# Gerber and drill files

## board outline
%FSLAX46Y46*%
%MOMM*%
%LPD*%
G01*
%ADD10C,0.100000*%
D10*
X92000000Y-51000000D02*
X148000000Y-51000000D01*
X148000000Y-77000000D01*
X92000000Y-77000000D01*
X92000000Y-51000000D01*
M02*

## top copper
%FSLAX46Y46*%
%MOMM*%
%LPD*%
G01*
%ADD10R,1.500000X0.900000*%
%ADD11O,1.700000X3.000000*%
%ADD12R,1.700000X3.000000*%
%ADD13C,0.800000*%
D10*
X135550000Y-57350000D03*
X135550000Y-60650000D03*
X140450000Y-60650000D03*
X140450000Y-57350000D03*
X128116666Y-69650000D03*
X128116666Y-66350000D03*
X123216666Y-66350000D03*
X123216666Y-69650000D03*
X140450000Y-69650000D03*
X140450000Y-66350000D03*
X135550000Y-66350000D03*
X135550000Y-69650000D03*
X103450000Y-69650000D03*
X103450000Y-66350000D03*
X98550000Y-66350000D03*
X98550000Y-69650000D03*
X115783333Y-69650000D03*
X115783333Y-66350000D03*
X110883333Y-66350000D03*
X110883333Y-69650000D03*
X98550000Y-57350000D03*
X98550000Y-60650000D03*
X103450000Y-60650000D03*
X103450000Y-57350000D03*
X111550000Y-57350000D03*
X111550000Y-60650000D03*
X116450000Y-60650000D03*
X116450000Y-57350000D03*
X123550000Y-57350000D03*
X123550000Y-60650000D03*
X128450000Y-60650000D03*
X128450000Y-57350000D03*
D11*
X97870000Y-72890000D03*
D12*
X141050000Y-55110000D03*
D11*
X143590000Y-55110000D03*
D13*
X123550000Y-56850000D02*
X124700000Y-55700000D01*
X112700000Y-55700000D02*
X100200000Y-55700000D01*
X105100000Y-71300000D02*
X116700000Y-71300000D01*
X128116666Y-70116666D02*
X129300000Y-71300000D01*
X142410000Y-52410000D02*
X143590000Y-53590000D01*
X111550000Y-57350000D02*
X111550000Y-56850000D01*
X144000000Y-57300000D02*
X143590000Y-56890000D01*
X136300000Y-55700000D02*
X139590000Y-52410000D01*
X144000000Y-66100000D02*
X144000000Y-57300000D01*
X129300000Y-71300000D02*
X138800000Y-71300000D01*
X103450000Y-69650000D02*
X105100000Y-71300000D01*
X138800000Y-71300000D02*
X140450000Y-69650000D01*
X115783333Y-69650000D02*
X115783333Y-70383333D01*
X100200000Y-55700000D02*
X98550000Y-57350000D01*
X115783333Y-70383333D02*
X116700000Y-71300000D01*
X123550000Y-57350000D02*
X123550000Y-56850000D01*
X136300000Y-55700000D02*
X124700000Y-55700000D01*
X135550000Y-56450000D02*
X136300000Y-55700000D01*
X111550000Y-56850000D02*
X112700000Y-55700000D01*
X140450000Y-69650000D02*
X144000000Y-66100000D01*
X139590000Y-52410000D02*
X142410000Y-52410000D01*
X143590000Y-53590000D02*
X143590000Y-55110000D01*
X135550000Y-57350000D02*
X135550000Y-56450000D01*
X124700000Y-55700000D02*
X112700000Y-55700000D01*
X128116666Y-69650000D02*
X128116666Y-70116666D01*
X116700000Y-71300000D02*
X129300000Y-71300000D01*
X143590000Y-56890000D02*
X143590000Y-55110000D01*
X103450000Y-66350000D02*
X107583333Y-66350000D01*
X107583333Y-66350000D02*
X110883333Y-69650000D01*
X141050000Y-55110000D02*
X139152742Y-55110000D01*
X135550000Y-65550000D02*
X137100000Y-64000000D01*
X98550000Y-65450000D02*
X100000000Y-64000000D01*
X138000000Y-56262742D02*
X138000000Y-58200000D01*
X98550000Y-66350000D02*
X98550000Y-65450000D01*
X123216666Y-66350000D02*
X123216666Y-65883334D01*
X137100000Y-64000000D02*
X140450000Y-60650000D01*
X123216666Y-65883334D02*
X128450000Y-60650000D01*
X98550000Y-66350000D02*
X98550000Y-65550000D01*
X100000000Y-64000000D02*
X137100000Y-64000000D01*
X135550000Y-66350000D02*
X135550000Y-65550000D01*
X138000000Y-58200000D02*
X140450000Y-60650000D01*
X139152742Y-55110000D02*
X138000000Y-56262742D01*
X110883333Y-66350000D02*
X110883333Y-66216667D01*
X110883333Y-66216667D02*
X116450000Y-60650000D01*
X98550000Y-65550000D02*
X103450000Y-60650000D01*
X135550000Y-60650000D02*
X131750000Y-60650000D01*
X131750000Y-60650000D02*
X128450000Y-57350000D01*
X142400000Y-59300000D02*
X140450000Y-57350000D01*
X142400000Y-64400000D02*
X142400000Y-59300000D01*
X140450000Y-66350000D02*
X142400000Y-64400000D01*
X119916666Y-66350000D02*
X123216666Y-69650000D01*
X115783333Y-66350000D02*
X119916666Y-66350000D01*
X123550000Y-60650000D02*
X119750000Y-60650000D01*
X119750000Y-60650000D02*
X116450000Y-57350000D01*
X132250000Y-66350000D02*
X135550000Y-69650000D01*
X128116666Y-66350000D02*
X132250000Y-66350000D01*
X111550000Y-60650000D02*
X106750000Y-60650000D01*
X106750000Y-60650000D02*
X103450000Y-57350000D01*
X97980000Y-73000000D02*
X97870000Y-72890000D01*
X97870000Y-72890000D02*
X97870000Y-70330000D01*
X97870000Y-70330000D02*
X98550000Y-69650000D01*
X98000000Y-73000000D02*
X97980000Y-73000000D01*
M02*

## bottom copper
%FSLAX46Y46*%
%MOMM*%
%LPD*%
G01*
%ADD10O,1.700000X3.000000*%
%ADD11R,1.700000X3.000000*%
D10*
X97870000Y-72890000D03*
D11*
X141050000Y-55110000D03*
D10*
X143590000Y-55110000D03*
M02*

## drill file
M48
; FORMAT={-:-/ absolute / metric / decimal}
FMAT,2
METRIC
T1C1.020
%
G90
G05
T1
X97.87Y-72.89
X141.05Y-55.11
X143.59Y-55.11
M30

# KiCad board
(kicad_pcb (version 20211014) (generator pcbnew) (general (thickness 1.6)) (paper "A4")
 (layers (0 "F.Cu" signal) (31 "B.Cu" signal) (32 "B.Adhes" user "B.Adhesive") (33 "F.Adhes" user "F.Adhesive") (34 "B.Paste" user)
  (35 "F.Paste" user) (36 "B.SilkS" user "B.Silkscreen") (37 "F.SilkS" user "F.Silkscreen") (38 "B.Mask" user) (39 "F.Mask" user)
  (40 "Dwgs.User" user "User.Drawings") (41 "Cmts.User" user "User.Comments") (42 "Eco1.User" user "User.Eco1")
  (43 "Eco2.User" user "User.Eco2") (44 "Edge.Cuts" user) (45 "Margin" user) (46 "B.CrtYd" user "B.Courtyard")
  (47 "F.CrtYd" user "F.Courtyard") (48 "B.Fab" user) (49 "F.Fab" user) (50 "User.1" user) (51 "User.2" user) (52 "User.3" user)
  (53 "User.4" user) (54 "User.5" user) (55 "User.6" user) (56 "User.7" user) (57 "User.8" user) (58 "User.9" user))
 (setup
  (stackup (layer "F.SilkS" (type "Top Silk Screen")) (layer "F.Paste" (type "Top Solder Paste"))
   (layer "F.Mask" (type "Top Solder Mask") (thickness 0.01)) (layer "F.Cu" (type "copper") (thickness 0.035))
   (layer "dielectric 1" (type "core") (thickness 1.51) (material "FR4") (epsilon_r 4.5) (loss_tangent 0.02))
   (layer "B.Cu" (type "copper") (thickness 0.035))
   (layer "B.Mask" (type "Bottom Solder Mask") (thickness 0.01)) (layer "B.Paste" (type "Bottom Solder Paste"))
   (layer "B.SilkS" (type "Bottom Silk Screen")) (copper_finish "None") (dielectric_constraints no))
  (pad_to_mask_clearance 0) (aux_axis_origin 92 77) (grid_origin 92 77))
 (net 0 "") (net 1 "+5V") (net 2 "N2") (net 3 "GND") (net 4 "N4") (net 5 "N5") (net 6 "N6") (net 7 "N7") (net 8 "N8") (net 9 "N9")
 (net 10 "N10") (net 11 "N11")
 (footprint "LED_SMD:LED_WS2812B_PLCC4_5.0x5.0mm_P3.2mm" (layer "F.Cu") (at 138 59)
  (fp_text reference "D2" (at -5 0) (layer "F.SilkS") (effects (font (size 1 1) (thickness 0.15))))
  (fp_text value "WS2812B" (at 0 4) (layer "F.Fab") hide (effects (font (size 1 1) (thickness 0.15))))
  (pad "1" smd rect (at -2.45 -1.65) (size 1.5 0.9) (layers "F.Cu" "F.Paste" "F.Mask") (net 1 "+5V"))
  (pad "2" smd rect (at -2.45 1.65) (size 1.5 0.9) (layers "F.Cu" "F.Paste" "F.Mask") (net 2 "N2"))
  (pad "3" smd rect (at 2.45 1.65) (size 1.5 0.9) (layers "F.Cu" "F.Paste" "F.Mask") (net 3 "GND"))
  (pad "4" smd rect (at 2.45 -1.65) (size 1.5 0.9) (layers "F.Cu" "F.Paste" "F.Mask") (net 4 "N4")))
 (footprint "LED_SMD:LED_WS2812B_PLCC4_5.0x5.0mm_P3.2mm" (layer "F.Cu") (at 125.666666 68 180)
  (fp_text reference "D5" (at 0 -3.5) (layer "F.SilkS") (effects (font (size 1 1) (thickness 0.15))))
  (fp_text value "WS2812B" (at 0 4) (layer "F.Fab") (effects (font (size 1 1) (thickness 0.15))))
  (pad "1" smd rect (at -2.45 -1.65 180) (size 1.5 0.9) (layers "F.Cu" "F.Paste" "F.Mask") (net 1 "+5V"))
  (pad "2" smd rect (at -2.45 1.65 180) (size 1.5 0.9) (layers "F.Cu" "F.Paste" "F.Mask") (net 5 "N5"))
  (pad "3" smd rect (at 2.45 1.65 180) (size 1.5 0.9) (layers "F.Cu" "F.Paste" "F.Mask") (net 3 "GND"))
  (pad "4" smd rect (at 2.45 -1.65 180) (size 1.5 0.9) (layers "F.Cu" "F.Paste" "F.Mask") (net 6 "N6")))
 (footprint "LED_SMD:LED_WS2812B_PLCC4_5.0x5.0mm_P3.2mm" (layer "F.Cu") (at 138 68 180)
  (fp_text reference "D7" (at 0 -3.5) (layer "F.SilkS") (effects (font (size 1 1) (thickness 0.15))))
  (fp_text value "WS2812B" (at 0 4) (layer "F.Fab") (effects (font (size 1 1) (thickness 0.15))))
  (pad "1" smd rect (at -2.45 -1.65 180) (size 1.5 0.9) (layers "F.Cu" "F.Paste" "F.Mask") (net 1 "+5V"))
  (pad "2" smd rect (at -2.45 1.65 180) (size 1.5 0.9) (layers "F.Cu" "F.Paste" "F.Mask") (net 4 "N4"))
  (pad "3" smd rect (at 2.45 1.65 180) (size 1.5 0.9) (layers "F.Cu" "F.Paste" "F.Mask") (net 3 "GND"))
  (pad "4" smd rect (at 2.45 -1.65 180) (size 1.5 0.9) (layers "F.Cu" "F.Paste" "F.Mask") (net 5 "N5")))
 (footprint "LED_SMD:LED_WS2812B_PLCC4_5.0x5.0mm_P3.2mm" (layer "F.Cu") (at 101 68 180)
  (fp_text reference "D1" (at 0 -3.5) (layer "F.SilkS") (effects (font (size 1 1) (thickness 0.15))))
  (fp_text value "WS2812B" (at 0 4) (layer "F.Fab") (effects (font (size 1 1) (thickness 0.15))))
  (pad "1" smd rect (at -2.45 -1.65 180) (size 1.5 0.9) (layers "F.Cu" "F.Paste" "F.Mask") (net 1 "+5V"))
  (pad "2" smd rect (at -2.45 1.65 180) (size 1.5 0.9) (layers "F.Cu" "F.Paste" "F.Mask") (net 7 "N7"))
  (pad "3" smd rect (at 2.45 1.65 180) (size 1.5 0.9) (layers "F.Cu" "F.Paste" "F.Mask") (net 3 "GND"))
  (pad "4" smd rect (at 2.45 -1.65 180) (size 1.5 0.9) (layers "F.Cu" "F.Paste" "F.Mask") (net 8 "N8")))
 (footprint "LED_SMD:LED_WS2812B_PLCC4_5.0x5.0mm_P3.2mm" (layer "F.Cu") (at 113.333333 68 180)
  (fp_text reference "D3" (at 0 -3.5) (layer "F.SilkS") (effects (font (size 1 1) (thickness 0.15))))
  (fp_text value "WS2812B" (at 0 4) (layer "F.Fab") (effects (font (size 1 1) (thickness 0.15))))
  (pad "1" smd rect (at -2.45 -1.65 180) (size 1.5 0.9) (layers "F.Cu" "F.Paste" "F.Mask") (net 1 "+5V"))
  (pad "2" smd rect (at -2.45 1.65 180) (size 1.5 0.9) (layers "F.Cu" "F.Paste" "F.Mask") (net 6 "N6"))
  (pad "3" smd rect (at 2.45 1.65 180) (size 1.5 0.9) (layers "F.Cu" "F.Paste" "F.Mask") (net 3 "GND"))
  (pad "4" smd rect (at 2.45 -1.65 180) (size 1.5 0.9) (layers "F.Cu" "F.Paste" "F.Mask") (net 7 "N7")))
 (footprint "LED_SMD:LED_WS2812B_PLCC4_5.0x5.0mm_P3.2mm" (layer "F.Cu") (at 101 59)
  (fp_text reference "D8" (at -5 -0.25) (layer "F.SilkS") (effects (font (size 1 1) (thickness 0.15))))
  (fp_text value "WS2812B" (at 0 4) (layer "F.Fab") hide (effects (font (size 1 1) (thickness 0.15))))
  (pad "1" smd rect (at -2.45 -1.65) (size 1.5 0.9) (layers "F.Cu" "F.Paste" "F.Mask") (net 1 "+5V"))
  (pad "2" smd rect (at -2.45 1.65) (size 1.5 0.9) (layers "F.Cu" "F.Paste" "F.Mask") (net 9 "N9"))
  (pad "3" smd rect (at 2.45 1.65) (size 1.5 0.9) (layers "F.Cu" "F.Paste" "F.Mask") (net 3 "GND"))
  (pad "4" smd rect (at 2.45 -1.65) (size 1.5 0.9) (layers "F.Cu" "F.Paste" "F.Mask") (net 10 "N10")))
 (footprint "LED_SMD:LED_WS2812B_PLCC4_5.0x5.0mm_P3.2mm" (layer "F.Cu") (at 114 59)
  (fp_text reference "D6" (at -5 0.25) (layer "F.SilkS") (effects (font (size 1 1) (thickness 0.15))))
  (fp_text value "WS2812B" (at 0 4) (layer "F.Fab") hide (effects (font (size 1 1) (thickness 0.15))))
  (pad "1" smd rect (at -2.45 -1.65) (size 1.5 0.9) (layers "F.Cu" "F.Paste" "F.Mask") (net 1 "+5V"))
  (pad "2" smd rect (at -2.45 1.65) (size 1.5 0.9) (layers "F.Cu" "F.Paste" "F.Mask") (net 10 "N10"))
  (pad "3" smd rect (at 2.45 1.65) (size 1.5 0.9) (layers "F.Cu" "F.Paste" "F.Mask") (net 3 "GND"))
  (pad "4" smd rect (at 2.45 -1.65) (size 1.5 0.9) (layers "F.Cu" "F.Paste" "F.Mask") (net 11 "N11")))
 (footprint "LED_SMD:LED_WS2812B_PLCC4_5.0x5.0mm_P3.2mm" (layer "F.Cu") (at 126 59)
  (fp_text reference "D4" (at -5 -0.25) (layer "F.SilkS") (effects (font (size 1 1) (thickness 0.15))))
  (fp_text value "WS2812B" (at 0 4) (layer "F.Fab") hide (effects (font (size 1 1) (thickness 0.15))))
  (pad "1" smd rect (at -2.45 -1.65) (size 1.5 0.9) (layers "F.Cu" "F.Paste" "F.Mask") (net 1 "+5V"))
  (pad "2" smd rect (at -2.45 1.65) (size 1.5 0.9) (layers "F.Cu" "F.Paste" "F.Mask") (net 11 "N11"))
  (pad "3" smd rect (at 2.45 1.65) (size 1.5 0.9) (layers "F.Cu" "F.Paste" "F.Mask") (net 3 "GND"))
  (pad "4" smd rect (at 2.45 -1.65) (size 1.5 0.9) (layers "F.Cu" "F.Paste" "F.Mask") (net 2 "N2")))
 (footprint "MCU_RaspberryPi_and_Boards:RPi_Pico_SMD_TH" (layer "B.Cu") (at 122 64 90)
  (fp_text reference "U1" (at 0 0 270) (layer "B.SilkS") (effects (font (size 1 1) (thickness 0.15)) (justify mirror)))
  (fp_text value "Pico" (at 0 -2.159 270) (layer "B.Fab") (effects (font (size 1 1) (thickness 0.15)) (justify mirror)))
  (pad "20" thru_hole oval (at -8.89 -24.13 90) (size 3 1.7) (drill 1.02) (layers *.Cu *.Mask) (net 8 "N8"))
  (pad "38" thru_hole rect (at 8.89 19.05 90) (size 3 1.7) (drill 1.02) (layers *.Cu *.Mask) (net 3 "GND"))
  (pad "39" thru_hole oval (at 8.89 21.59 90) (size 3 1.7) (drill 1.02) (layers *.Cu *.Mask) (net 1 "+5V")))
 (gr_rect (start 92 51) (end 148 77) (layer "Edge.Cuts") (width 0.1) (fill none))
 (segment (start 123.55 56.85) (end 124.7 55.7) (width 0.8) (layer "F.Cu") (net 1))
 (segment (start 112.7 55.7) (end 100.2 55.7) (width 0.8) (layer "F.Cu") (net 1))
 (segment (start 105.1 71.3) (end 116.7 71.3) (width 0.8) (layer "F.Cu") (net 1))
 (segment (start 128.116666 70.116666) (end 129.3 71.3) (width 0.8) (layer "F.Cu") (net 1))
 (segment (start 142.41 52.41) (end 143.59 53.59) (width 0.8) (layer "F.Cu") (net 1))
 (segment (start 111.55 57.35) (end 111.55 56.85) (width 0.8) (layer "F.Cu") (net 1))
 (segment (start 144 57.3) (end 143.59 56.89) (width 0.8) (layer "F.Cu") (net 1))
 (segment (start 136.3 55.7) (end 139.59 52.41) (width 0.8) (layer "F.Cu") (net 1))
 (segment (start 144 66.1) (end 144 57.3) (width 0.8) (layer "F.Cu") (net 1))
 (segment (start 129.3 71.3) (end 138.8 71.3) (width 0.8) (layer "F.Cu") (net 1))
 (segment (start 103.45 69.65) (end 105.1 71.3) (width 0.8) (layer "F.Cu") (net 1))
 (segment (start 138.8 71.3) (end 140.45 69.65) (width 0.8) (layer "F.Cu") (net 1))
 (segment (start 115.783333 69.65) (end 115.783333 70.383333) (width 0.8) (layer "F.Cu") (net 1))
 (segment (start 100.2 55.7) (end 98.55 57.35) (width 0.8) (layer "F.Cu") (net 1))
 (segment (start 115.783333 70.383333) (end 116.7 71.3) (width 0.8) (layer "F.Cu") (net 1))
 (segment (start 123.55 57.35) (end 123.55 56.85) (width 0.8) (layer "F.Cu") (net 1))
 (segment (start 136.3 55.7) (end 124.7 55.7) (width 0.8) (layer "F.Cu") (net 1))
 (segment (start 135.55 56.45) (end 136.3 55.7) (width 0.8) (layer "F.Cu") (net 1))
 (segment (start 111.55 56.85) (end 112.7 55.7) (width 0.8) (layer "F.Cu") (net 1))
 (segment (start 140.45 69.65) (end 144 66.1) (width 0.8) (layer "F.Cu") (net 1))
 (segment (start 139.59 52.41) (end 142.41 52.41) (width 0.8) (layer "F.Cu") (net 1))
 (segment (start 143.59 53.59) (end 143.59 55.11) (width 0.8) (layer "F.Cu") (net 1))
 (segment (start 135.55 57.35) (end 135.55 56.45) (width 0.8) (layer "F.Cu") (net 1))
 (segment (start 124.7 55.7) (end 112.7 55.7) (width 0.8) (layer "F.Cu") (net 1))
 (segment (start 128.116666 69.65) (end 128.116666 70.116666) (width 0.8) (layer "F.Cu") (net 1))
 (segment (start 116.7 71.3) (end 129.3 71.3) (width 0.8) (layer "F.Cu") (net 1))
 (segment (start 143.59 56.89) (end 143.59 55.11) (width 0.8) (layer "F.Cu") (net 1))
 (segment (start 103.45 66.35) (end 107.583333 66.35) (width 0.8) (layer "F.Cu") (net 7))
 (segment (start 107.583333 66.35) (end 110.883333 69.65) (width 0.8) (layer "F.Cu") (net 7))
 (segment (start 141.05 55.11) (end 139.152742 55.11) (width 0.8) (layer "F.Cu") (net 3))
 (segment (start 135.55 65.55) (end 137.1 64) (width 0.8) (layer "F.Cu") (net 3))
 (segment (start 98.55 65.45) (end 100 64) (width 0.8) (layer "F.Cu") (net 3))
 (segment (start 138 56.262742) (end 138 58.2) (width 0.8) (layer "F.Cu") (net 3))
 (segment (start 98.55 66.35) (end 98.55 65.45) (width 0.8) (layer "F.Cu") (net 3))
 (segment (start 123.216666 66.35) (end 123.216666 65.883334) (width 0.8) (layer "F.Cu") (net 3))
 (segment (start 137.1 64) (end 140.45 60.65) (width 0.8) (layer "F.Cu") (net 3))
 (segment (start 123.216666 65.883334) (end 128.45 60.65) (width 0.8) (layer "F.Cu") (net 3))
 (segment (start 98.55 66.35) (end 98.55 65.55) (width 0.8) (layer "F.Cu") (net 3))
 (segment (start 100 64) (end 137.1 64) (width 0.8) (layer "F.Cu") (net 3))
 (segment (start 135.55 66.35) (end 135.55 65.55) (width 0.8) (layer "F.Cu") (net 3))
 (segment (start 138 58.2) (end 140.45 60.65) (width 0.8) (layer "F.Cu") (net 3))
 (segment (start 139.152742 55.11) (end 138 56.262742) (width 0.8) (layer "F.Cu") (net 3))
 (segment (start 110.883333 66.35) (end 110.883333 66.216667) (width 0.8) (layer "F.Cu") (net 3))
 (segment (start 110.883333 66.216667) (end 116.45 60.65) (width 0.8) (layer "F.Cu") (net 3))
 (segment (start 98.55 65.55) (end 103.45 60.65) (width 0.8) (layer "F.Cu") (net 3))
 (segment (start 135.55 60.65) (end 131.75 60.65) (width 0.8) (layer "F.Cu") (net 2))
 (segment (start 131.75 60.65) (end 128.45 57.35) (width 0.8) (layer "F.Cu") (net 2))
 (segment (start 142.4 59.3) (end 140.45 57.35) (width 0.8) (layer "F.Cu") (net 4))
 (segment (start 142.4 64.4) (end 142.4 59.3) (width 0.8) (layer "F.Cu") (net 4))
 (segment (start 140.45 66.35) (end 142.4 64.4) (width 0.8) (layer "F.Cu") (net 4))
 (segment (start 119.916666 66.35) (end 123.216666 69.65) (width 0.8) (layer "F.Cu") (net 6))
 (segment (start 115.783333 66.35) (end 119.916666 66.35) (width 0.8) (layer "F.Cu") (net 6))
 (segment (start 123.55 60.65) (end 119.75 60.65) (width 0.8) (layer "F.Cu") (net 11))
 (segment (start 119.75 60.65) (end 116.45 57.35) (width 0.8) (layer "F.Cu") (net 11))
 (segment (start 132.25 66.35) (end 135.55 69.65) (width 0.8) (layer "F.Cu") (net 5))
 (segment (start 128.116666 66.35) (end 132.25 66.35) (width 0.8) (layer "F.Cu") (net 5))
 (segment (start 111.55 60.65) (end 106.75 60.65) (width 0.8) (layer "F.Cu") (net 10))
 (segment (start 106.75 60.65) (end 103.45 57.35) (width 0.8) (layer "F.Cu") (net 10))
 (segment (start 97.98 73) (end 97.87 72.89) (width 0.8) (layer "F.Cu") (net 8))
 (segment (start 97.87 72.89) (end 97.87 70.33) (width 0.8) (layer "F.Cu") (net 8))
 (segment (start 97.87 70.33) (end 98.55 69.65) (width 0.8) (layer "F.Cu") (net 8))
 (segment (start 98 73) (end 97.98 73) (width 0.8) (layer "F.Cu") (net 8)))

